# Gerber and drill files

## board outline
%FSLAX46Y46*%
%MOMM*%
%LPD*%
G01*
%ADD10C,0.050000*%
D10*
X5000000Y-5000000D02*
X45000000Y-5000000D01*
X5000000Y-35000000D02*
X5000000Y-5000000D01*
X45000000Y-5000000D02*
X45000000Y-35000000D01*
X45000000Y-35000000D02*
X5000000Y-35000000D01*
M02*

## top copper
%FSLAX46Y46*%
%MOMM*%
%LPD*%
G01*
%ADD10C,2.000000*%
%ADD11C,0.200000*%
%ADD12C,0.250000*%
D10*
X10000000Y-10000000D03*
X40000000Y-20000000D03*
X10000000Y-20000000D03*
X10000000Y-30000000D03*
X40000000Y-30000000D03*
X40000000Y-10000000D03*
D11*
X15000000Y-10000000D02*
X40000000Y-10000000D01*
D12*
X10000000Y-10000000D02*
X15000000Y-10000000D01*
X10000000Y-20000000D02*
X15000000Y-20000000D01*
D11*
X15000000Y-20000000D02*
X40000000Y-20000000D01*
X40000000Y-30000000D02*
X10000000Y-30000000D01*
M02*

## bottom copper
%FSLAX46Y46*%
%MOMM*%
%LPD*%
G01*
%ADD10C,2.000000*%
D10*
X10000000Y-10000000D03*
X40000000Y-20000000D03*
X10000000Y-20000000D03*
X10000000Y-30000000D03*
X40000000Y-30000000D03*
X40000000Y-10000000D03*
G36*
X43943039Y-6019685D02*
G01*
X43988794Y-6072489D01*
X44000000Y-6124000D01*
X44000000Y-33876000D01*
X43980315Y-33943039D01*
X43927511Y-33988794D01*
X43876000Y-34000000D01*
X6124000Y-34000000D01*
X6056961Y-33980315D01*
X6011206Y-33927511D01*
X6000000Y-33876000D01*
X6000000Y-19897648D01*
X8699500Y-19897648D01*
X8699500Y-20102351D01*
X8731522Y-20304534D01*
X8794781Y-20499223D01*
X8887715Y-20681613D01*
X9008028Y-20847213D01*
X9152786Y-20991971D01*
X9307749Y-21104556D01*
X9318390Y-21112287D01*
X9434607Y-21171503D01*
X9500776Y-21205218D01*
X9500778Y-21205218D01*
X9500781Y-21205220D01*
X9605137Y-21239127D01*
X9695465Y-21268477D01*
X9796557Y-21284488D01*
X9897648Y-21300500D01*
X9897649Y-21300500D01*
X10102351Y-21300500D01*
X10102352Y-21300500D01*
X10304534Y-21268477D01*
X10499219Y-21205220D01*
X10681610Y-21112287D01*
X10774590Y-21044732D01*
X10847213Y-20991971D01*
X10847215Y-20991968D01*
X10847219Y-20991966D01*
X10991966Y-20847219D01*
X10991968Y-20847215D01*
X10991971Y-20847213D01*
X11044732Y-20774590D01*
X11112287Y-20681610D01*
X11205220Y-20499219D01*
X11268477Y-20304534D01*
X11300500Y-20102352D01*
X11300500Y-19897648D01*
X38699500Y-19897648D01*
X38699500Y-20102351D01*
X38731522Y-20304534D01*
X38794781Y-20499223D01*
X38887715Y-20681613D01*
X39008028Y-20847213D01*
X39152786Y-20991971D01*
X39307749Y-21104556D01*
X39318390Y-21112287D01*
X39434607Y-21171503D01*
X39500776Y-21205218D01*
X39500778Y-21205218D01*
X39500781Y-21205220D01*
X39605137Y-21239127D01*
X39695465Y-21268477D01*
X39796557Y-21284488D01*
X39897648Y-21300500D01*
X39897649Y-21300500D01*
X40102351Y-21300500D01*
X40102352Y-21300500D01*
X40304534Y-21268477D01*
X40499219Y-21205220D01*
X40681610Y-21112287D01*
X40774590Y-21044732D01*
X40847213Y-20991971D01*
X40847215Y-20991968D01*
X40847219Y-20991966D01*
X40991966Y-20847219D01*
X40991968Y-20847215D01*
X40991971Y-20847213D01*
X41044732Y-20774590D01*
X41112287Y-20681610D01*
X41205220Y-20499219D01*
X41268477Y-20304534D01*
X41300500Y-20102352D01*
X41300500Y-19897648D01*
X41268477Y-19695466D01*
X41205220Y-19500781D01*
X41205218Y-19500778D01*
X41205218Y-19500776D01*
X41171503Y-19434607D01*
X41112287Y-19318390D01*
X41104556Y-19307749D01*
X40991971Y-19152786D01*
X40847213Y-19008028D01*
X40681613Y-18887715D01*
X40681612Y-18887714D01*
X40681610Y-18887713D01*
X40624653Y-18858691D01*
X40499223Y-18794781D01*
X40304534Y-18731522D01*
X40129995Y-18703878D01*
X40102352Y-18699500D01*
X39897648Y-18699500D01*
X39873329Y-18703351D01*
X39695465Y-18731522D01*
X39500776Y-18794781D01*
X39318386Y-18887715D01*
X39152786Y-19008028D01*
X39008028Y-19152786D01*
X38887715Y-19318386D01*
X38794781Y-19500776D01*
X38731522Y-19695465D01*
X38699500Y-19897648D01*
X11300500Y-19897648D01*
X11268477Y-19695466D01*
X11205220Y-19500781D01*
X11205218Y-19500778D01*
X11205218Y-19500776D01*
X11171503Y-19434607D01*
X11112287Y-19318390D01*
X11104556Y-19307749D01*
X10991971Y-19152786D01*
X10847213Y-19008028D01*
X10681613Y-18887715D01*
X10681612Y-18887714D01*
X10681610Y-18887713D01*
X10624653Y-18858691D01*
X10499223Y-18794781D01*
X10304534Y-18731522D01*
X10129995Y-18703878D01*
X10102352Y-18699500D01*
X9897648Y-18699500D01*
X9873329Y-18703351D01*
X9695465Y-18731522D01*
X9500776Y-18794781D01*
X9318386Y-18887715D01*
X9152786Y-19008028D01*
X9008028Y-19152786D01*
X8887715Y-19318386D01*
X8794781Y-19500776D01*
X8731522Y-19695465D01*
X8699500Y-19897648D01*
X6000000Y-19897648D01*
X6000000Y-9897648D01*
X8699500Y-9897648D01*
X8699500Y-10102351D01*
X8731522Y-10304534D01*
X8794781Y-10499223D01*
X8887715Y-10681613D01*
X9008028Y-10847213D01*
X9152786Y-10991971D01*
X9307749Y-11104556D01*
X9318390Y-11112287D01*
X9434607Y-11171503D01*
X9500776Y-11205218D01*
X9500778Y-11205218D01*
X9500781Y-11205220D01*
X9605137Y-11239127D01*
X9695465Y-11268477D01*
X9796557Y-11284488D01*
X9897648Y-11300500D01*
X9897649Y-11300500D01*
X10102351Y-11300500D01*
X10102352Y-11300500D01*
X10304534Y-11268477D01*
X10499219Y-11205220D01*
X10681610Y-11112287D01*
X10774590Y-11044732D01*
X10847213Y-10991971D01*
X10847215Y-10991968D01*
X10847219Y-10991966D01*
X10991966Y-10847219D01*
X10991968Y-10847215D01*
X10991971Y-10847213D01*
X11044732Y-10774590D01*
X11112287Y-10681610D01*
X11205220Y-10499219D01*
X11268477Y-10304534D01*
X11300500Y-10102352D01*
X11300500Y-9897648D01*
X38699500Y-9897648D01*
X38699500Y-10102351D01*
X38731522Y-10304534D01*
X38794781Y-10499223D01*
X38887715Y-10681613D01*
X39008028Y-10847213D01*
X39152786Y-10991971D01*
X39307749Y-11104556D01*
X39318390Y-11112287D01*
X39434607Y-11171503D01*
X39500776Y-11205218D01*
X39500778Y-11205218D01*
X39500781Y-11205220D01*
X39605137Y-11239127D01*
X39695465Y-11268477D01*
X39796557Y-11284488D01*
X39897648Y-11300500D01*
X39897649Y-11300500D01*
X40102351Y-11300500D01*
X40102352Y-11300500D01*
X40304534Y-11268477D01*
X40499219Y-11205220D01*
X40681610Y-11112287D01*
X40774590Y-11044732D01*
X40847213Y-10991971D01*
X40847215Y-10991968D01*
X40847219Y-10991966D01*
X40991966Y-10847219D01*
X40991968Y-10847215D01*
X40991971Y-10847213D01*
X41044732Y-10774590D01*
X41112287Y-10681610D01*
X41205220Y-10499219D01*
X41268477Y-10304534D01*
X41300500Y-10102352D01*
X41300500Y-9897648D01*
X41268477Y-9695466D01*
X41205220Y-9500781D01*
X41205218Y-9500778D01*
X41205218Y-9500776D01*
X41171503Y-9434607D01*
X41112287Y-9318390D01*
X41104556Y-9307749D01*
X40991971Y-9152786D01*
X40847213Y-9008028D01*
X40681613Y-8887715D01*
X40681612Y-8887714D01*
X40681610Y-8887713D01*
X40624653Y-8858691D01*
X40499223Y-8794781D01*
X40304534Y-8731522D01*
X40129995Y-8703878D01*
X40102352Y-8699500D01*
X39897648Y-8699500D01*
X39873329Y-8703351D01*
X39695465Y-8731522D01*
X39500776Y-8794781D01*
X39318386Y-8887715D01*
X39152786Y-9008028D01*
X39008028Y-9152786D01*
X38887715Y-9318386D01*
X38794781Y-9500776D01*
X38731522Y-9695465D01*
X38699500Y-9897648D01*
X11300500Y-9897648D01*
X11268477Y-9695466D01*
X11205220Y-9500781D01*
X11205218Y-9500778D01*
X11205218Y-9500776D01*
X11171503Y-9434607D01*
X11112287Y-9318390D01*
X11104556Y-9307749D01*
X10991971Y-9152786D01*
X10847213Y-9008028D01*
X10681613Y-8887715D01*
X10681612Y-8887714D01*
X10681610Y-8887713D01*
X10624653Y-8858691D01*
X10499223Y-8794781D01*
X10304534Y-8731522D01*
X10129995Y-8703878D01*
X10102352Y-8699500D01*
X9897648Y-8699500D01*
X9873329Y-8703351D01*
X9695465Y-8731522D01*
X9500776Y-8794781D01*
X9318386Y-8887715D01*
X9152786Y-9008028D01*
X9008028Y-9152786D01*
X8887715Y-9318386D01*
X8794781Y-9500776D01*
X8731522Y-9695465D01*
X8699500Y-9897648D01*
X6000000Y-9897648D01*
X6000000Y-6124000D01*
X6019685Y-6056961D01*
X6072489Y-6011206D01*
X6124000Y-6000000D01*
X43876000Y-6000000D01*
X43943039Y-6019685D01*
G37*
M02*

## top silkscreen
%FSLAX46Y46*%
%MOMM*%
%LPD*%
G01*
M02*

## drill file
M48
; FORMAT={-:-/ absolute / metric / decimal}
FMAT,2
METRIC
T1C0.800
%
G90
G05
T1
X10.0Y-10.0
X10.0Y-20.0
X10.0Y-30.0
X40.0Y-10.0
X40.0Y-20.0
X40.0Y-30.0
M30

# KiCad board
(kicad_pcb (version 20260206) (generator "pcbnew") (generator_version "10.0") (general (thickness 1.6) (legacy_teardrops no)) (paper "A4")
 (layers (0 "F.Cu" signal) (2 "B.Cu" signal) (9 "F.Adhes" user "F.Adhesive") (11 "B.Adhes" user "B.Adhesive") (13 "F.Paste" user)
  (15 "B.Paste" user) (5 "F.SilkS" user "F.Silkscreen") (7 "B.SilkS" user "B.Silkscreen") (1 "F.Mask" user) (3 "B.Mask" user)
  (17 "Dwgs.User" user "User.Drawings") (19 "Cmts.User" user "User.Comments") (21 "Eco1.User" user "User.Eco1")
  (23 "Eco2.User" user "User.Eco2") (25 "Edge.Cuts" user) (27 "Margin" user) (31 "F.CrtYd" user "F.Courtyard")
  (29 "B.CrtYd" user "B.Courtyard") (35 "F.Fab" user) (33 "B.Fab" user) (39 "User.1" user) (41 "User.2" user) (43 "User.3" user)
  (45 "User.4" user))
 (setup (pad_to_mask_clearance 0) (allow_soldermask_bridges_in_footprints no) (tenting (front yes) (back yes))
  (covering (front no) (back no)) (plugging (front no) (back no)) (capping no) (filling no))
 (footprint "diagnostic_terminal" (layer "F.Cu") (at 10 10)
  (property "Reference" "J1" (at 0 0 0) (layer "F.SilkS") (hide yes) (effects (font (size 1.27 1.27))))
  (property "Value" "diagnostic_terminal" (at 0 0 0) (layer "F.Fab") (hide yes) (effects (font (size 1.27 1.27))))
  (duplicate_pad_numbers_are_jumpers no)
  (pad "1" thru_hole circle (at 0 0) (size 2 2) (drill 0.8) (layers "*.Cu") (remove_unused_layers no) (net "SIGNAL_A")))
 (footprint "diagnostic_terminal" (layer "F.Cu") (at 40 20)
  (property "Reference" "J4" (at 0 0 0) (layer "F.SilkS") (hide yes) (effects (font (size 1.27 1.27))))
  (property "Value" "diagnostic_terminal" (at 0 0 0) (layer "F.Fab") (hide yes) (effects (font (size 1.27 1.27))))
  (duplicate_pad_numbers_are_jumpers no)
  (pad "1" thru_hole circle (at 0 0) (size 2 2) (drill 0.8) (layers "*.Cu") (remove_unused_layers no) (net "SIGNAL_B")))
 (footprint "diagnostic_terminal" (layer "F.Cu") (at 10 20)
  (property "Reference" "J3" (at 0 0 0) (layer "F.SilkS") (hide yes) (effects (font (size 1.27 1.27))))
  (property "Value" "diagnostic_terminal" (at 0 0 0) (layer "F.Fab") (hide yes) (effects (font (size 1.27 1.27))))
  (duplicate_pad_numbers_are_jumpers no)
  (pad "1" thru_hole circle (at 0 0) (size 2 2) (drill 0.8) (layers "*.Cu") (remove_unused_layers no) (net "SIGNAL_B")))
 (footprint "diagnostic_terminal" (layer "F.Cu") (at 10 30)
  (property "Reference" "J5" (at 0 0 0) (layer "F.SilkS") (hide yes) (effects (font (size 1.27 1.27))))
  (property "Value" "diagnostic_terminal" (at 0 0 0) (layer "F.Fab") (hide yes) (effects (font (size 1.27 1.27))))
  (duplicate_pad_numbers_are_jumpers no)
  (pad "1" thru_hole circle (at 0 0) (size 2 2) (drill 0.8) (layers "*.Cu") (remove_unused_layers no) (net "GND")))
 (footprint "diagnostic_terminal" (layer "F.Cu") (at 40 30)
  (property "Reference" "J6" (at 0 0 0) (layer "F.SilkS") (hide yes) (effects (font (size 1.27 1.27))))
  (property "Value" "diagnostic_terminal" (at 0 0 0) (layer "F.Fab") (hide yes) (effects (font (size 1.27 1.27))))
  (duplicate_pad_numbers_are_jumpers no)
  (pad "1" thru_hole circle (at 0 0) (size 2 2) (drill 0.8) (layers "*.Cu") (remove_unused_layers no) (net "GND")))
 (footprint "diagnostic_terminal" (layer "F.Cu") (at 40 10)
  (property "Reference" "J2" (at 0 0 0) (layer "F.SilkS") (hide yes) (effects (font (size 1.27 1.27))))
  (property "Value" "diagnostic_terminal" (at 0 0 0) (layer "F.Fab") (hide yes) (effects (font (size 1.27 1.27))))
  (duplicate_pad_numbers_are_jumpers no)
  (pad "1" thru_hole circle (at 0 0) (size 2 2) (drill 0.8) (layers "*.Cu") (remove_unused_layers no) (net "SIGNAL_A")))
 (gr_line (start 5 5) (end 45 5) (stroke (width 0.05) (type default)) (layer "Edge.Cuts"))
 (gr_line (start 5 35) (end 5 5) (stroke (width 0.05) (type default)) (layer "Edge.Cuts"))
 (gr_line (start 45 5) (end 45 35) (stroke (width 0.05) (type default)) (layer "Edge.Cuts"))
 (gr_line (start 45 35) (end 5 35) (stroke (width 0.05) (type default)) (layer "Edge.Cuts"))
 (segment (start 15 10) (end 40 10) (width 0.2) (layer "F.Cu") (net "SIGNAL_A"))
 (segment (start 10 10) (end 15 10) (width 0.25) (locked yes) (layer "F.Cu") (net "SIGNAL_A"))
 (segment (start 10 20) (end 15 20) (width 0.25) (locked yes) (layer "F.Cu") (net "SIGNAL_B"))
 (segment (start 15 20) (end 40 20) (width 0.2) (layer "F.Cu") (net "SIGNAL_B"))
 (segment (start 40 30) (end 10 30) (width 0.2) (layer "F.Cu") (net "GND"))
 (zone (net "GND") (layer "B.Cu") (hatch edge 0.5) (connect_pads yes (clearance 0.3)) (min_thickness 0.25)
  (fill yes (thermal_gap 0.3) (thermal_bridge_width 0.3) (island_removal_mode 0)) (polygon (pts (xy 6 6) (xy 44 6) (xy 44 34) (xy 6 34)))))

